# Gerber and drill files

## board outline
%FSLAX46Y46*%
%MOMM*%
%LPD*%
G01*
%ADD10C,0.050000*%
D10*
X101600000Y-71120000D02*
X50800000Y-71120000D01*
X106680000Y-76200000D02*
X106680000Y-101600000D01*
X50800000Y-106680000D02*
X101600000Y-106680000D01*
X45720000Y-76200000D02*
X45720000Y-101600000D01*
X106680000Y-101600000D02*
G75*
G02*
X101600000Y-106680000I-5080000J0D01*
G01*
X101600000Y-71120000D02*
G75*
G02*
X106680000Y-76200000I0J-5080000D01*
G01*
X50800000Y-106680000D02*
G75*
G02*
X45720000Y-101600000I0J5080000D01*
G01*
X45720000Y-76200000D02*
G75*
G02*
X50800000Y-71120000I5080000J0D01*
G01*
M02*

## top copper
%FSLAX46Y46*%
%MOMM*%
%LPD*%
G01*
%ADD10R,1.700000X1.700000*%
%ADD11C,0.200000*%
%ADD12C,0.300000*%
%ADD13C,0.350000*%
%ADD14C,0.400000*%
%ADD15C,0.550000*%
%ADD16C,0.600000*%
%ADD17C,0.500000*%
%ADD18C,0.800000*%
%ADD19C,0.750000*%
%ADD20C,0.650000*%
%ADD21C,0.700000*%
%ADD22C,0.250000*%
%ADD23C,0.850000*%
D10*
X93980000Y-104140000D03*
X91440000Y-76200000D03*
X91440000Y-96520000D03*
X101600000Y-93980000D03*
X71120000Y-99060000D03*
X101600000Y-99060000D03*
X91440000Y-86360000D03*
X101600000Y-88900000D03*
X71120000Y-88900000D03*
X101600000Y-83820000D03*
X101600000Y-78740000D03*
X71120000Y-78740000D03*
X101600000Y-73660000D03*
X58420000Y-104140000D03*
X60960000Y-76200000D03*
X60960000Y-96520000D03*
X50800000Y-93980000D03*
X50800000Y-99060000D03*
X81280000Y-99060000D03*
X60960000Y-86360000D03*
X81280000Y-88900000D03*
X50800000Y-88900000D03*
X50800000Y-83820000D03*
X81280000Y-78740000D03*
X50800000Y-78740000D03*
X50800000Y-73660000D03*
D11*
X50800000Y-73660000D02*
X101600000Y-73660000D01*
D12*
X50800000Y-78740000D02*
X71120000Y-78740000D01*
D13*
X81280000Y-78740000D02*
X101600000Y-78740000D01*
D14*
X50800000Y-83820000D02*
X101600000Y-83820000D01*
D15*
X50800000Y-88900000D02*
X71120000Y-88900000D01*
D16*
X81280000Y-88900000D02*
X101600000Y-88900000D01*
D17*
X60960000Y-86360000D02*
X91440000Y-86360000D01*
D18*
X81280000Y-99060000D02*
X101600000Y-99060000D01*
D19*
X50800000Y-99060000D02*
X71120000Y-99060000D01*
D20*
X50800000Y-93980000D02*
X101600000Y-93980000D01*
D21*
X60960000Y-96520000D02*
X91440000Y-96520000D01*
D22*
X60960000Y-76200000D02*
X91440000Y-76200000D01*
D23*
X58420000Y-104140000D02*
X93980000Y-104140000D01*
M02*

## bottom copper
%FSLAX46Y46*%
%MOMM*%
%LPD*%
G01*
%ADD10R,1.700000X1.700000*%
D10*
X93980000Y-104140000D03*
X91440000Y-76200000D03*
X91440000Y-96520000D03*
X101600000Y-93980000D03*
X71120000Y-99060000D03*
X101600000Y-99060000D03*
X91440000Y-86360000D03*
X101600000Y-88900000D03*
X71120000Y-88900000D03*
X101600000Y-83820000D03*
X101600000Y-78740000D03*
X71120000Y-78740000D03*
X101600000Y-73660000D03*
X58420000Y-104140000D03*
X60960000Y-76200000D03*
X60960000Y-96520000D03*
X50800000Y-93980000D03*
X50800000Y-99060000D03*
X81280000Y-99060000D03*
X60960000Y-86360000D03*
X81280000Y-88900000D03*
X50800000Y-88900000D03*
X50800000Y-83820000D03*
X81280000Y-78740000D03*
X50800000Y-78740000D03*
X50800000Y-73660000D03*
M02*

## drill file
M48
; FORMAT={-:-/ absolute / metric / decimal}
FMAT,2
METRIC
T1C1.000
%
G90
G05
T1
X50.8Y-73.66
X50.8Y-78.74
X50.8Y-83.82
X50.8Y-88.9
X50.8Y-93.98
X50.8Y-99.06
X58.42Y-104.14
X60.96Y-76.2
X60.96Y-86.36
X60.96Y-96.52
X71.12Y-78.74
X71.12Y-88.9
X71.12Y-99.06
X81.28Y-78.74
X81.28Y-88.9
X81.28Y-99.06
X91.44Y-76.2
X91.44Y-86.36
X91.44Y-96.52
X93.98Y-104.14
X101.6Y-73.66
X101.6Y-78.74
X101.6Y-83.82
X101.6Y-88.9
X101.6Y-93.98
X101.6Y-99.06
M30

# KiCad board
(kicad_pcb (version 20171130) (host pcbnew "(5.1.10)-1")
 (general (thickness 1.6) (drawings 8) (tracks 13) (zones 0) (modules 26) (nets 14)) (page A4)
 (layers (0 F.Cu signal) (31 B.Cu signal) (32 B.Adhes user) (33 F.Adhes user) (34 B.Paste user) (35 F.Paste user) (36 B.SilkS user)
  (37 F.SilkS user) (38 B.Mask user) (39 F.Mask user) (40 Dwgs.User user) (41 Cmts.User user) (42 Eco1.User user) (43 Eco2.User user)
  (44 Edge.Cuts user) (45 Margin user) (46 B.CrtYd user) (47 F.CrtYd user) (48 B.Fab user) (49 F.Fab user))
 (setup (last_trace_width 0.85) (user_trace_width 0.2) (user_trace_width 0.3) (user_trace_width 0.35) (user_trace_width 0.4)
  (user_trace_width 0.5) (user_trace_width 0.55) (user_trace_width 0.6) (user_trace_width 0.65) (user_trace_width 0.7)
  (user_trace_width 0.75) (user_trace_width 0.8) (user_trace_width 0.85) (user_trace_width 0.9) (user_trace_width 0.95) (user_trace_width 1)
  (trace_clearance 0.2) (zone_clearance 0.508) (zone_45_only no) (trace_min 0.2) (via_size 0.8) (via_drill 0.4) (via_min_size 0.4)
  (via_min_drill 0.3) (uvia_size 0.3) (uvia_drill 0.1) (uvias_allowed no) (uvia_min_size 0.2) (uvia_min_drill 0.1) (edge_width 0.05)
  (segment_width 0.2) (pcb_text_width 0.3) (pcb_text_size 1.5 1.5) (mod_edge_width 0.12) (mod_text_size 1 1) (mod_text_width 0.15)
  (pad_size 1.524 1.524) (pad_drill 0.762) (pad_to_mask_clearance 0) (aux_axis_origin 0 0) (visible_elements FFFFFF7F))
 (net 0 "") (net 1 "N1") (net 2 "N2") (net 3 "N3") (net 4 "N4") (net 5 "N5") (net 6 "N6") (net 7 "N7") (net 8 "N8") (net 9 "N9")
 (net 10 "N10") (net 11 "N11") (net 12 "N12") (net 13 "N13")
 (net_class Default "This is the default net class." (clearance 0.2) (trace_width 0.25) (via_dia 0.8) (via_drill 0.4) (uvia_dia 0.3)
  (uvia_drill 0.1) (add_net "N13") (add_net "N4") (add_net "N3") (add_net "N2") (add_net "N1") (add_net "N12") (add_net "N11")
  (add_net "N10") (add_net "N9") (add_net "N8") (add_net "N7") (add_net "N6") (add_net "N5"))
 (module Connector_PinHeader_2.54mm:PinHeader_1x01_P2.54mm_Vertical (layer F.Cu) (at 93.98 104.14)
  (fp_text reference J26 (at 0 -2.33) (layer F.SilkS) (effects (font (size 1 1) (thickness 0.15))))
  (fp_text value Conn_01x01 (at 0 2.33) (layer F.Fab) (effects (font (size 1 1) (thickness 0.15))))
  (pad 1 thru_hole rect (at 0 0) (size 1.7 1.7) (drill 1) (layers *.Cu *.Mask) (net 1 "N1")))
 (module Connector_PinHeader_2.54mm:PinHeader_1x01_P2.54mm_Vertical (layer F.Cu) (at 91.44 76.2)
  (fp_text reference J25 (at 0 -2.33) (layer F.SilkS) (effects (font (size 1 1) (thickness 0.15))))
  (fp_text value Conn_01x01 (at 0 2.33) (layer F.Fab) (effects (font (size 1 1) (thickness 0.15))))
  (pad 1 thru_hole rect (at 0 0) (size 1.7 1.7) (drill 1) (layers *.Cu *.Mask) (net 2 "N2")))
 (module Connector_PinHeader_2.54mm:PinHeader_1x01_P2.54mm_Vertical (layer F.Cu) (at 91.44 96.52)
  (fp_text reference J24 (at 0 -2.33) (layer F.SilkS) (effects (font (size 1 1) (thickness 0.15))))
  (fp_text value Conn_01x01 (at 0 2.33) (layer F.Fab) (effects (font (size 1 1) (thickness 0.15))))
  (pad 1 thru_hole rect (at 0 0) (size 1.7 1.7) (drill 1) (layers *.Cu *.Mask) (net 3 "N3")))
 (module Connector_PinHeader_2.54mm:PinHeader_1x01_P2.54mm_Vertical (layer F.Cu) (at 101.6 93.98)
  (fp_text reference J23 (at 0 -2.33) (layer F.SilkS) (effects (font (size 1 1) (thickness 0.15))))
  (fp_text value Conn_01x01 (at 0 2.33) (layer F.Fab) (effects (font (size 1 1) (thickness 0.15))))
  (pad 1 thru_hole rect (at 0 0) (size 1.7 1.7) (drill 1) (layers *.Cu *.Mask) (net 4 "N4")))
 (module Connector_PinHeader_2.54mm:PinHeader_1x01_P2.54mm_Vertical (layer F.Cu) (at 71.12 99.06)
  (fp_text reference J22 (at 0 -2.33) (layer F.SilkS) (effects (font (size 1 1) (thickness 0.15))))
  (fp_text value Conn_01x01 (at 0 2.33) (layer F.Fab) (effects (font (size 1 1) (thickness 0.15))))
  (pad 1 thru_hole rect (at 0 0) (size 1.7 1.7) (drill 1) (layers *.Cu *.Mask) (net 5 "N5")))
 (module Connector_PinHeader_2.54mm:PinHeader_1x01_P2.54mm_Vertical (layer F.Cu) (at 101.6 99.06)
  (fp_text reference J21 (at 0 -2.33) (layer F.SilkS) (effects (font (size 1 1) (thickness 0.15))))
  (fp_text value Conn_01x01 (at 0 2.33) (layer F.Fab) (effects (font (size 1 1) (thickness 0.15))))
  (pad 1 thru_hole rect (at 0 0) (size 1.7 1.7) (drill 1) (layers *.Cu *.Mask) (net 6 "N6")))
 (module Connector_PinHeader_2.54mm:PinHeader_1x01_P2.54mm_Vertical (layer F.Cu) (at 91.44 86.36)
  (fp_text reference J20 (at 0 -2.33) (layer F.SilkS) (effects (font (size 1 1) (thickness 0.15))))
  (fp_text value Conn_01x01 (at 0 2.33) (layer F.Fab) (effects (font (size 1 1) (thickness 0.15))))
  (pad 1 thru_hole rect (at 0 0) (size 1.7 1.7) (drill 1) (layers *.Cu *.Mask) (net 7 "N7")))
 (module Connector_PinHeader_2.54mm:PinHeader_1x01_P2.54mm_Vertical (layer F.Cu) (at 101.6 88.9)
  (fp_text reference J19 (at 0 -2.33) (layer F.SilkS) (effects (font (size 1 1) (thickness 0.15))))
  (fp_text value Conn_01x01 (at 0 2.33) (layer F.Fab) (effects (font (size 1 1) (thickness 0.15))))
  (pad 1 thru_hole rect (at 0 0) (size 1.7 1.7) (drill 1) (layers *.Cu *.Mask) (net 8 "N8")))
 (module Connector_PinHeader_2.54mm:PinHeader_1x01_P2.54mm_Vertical (layer F.Cu) (at 71.12 88.9)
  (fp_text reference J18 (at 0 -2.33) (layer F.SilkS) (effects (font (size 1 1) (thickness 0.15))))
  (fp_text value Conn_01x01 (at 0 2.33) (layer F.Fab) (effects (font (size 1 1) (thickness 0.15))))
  (pad 1 thru_hole rect (at 0 0) (size 1.7 1.7) (drill 1) (layers *.Cu *.Mask) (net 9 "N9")))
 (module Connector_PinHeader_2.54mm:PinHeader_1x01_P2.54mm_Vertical (layer F.Cu) (at 101.6 83.82)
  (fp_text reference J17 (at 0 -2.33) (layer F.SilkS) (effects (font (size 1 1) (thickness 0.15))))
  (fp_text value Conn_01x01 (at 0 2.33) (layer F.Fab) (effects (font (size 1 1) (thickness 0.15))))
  (pad 1 thru_hole rect (at 0 0) (size 1.7 1.7) (drill 1) (layers *.Cu *.Mask) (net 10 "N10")))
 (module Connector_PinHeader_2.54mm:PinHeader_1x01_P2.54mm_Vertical (layer F.Cu) (at 101.6 78.74)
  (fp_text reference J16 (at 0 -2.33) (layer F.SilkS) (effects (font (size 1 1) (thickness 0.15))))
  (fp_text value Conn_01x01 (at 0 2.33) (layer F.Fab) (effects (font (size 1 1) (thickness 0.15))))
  (pad 1 thru_hole rect (at 0 0) (size 1.7 1.7) (drill 1) (layers *.Cu *.Mask) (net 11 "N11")))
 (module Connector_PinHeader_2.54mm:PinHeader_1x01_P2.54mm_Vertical (layer F.Cu) (at 71.12 78.74)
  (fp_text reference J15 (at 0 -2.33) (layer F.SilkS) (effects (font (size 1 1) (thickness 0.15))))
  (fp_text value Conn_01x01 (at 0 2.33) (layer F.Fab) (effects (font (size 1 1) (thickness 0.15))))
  (pad 1 thru_hole rect (at 0 0) (size 1.7 1.7) (drill 1) (layers *.Cu *.Mask) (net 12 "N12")))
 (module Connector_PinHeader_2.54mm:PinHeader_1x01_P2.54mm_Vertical (layer F.Cu) (at 101.6 73.66)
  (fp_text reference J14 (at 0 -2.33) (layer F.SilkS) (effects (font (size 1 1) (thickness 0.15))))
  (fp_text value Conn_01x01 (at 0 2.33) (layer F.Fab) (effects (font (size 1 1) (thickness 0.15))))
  (pad 1 thru_hole rect (at 0 0) (size 1.7 1.7) (drill 1) (layers *.Cu *.Mask) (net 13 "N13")))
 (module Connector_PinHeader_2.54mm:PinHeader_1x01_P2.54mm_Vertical (layer F.Cu) (at 58.42 104.14)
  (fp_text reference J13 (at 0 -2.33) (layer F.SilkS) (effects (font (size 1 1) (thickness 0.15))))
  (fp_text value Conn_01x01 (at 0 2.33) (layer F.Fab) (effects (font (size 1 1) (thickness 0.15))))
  (pad 1 thru_hole rect (at 0 0) (size 1.7 1.7) (drill 1) (layers *.Cu *.Mask) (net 1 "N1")))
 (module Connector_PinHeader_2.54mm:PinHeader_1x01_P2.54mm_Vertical (layer F.Cu) (at 60.96 76.2)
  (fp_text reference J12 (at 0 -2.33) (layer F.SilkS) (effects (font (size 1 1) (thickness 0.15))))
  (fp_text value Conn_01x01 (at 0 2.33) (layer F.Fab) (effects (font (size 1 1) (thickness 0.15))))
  (pad 1 thru_hole rect (at 0 0) (size 1.7 1.7) (drill 1) (layers *.Cu *.Mask) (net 2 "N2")))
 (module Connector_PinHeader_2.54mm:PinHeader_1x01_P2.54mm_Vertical (layer F.Cu) (at 60.96 96.52)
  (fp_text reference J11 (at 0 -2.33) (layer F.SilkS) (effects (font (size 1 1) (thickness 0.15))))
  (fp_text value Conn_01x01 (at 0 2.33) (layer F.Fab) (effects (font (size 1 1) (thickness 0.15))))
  (pad 1 thru_hole rect (at 0 0) (size 1.7 1.7) (drill 1) (layers *.Cu *.Mask) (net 3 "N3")))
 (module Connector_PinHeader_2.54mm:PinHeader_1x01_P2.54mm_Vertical (layer F.Cu) (at 50.8 93.98)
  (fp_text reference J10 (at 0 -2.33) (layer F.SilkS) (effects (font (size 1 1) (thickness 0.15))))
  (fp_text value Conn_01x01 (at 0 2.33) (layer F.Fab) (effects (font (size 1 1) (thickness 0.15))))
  (pad 1 thru_hole rect (at 0 0) (size 1.7 1.7) (drill 1) (layers *.Cu *.Mask) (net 4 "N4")))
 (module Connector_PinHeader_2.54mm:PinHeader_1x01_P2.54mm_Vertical (layer F.Cu) (at 50.8 99.06)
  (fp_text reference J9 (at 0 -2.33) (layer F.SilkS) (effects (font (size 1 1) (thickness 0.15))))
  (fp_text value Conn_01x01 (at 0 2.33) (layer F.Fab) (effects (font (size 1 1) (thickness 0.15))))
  (pad 1 thru_hole rect (at 0 0) (size 1.7 1.7) (drill 1) (layers *.Cu *.Mask) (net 5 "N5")))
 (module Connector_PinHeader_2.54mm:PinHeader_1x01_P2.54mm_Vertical (layer F.Cu) (at 81.28 99.06)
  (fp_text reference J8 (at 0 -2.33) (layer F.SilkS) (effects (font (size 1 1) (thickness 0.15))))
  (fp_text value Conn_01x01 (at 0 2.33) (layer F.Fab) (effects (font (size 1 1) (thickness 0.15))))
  (pad 1 thru_hole rect (at 0 0) (size 1.7 1.7) (drill 1) (layers *.Cu *.Mask) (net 6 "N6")))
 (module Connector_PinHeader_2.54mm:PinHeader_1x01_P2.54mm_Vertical (layer F.Cu) (at 60.96 86.36)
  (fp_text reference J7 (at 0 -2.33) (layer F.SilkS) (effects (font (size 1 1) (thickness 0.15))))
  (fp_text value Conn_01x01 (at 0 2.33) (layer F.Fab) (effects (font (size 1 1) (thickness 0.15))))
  (pad 1 thru_hole rect (at 0 0) (size 1.7 1.7) (drill 1) (layers *.Cu *.Mask) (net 7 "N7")))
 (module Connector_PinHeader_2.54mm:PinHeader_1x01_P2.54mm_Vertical (layer F.Cu) (at 81.28 88.9)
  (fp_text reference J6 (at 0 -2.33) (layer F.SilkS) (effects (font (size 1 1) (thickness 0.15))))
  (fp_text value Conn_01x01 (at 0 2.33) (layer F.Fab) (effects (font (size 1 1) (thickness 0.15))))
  (pad 1 thru_hole rect (at 0 0) (size 1.7 1.7) (drill 1) (layers *.Cu *.Mask) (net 8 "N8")))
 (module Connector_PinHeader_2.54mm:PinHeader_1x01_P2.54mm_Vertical (layer F.Cu) (at 50.8 88.9)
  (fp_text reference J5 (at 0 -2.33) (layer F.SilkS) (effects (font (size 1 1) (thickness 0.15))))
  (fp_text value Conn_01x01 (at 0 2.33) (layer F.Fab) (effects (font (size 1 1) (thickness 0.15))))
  (pad 1 thru_hole rect (at 0 0) (size 1.7 1.7) (drill 1) (layers *.Cu *.Mask) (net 9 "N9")))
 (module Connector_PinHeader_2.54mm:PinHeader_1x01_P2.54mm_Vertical (layer F.Cu) (at 50.8 83.82)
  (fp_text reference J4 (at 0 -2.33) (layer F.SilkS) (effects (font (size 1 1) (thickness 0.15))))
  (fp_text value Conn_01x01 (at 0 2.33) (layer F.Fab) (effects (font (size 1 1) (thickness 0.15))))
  (pad 1 thru_hole rect (at 0 0) (size 1.7 1.7) (drill 1) (layers *.Cu *.Mask) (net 10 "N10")))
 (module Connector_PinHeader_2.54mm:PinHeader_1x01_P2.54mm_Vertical (layer F.Cu) (at 81.28 78.74)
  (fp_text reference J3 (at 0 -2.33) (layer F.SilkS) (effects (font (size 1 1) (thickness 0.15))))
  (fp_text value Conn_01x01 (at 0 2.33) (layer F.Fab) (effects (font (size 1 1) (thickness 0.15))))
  (pad 1 thru_hole rect (at 0 0) (size 1.7 1.7) (drill 1) (layers *.Cu *.Mask) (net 11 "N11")))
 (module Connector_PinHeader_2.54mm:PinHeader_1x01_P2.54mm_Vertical (layer F.Cu) (at 50.8 78.74)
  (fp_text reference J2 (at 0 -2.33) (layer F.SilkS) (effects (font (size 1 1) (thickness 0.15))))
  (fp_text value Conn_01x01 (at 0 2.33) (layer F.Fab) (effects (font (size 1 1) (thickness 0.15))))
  (pad 1 thru_hole rect (at 0 0) (size 1.7 1.7) (drill 1) (layers *.Cu *.Mask) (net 12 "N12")))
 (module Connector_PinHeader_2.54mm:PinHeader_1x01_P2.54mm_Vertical (layer F.Cu) (at 50.8 73.66)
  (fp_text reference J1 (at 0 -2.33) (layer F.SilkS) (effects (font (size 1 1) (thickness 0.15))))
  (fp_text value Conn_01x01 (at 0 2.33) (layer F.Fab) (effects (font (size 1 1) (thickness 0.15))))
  (pad 1 thru_hole rect (at 0 0) (size 1.7 1.7) (drill 1) (layers *.Cu *.Mask) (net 13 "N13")))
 (gr_line (start 101.6 71.12) (end 50.8 71.12) (layer Edge.Cuts) (width 0.05))
 (gr_line (start 106.68 76.2) (end 106.68 101.6) (layer Edge.Cuts) (width 0.05))
 (gr_line (start 50.8 106.68) (end 101.6 106.68) (layer Edge.Cuts) (width 0.05))
 (gr_line (start 45.72 76.2) (end 45.72 101.6) (layer Edge.Cuts) (width 0.05))
 (gr_arc (start 101.6 101.6) (end 101.6 106.68) (angle -90) (layer Edge.Cuts) (width 0.05))
 (gr_arc (start 101.6 76.2) (end 106.68 76.2) (angle -90) (layer Edge.Cuts) (width 0.05))
 (gr_arc (start 50.8 101.6) (end 45.72 101.6) (angle -90) (layer Edge.Cuts) (width 0.05))
 (gr_arc (start 50.8 76.2) (end 50.8 71.12) (angle -90) (layer Edge.Cuts) (width 0.05))
 (segment (start 50.8 73.66) (end 101.6 73.66) (width 0.2) (layer F.Cu) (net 13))
 (segment (start 50.8 78.74) (end 71.12 78.74) (width 0.3) (layer F.Cu) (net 12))
 (segment (start 81.28 78.74) (end 101.6 78.74) (width 0.35) (layer F.Cu) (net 11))
 (segment (start 50.8 83.82) (end 101.6 83.82) (width 0.4) (layer F.Cu) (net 10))
 (segment (start 50.8 88.9) (end 71.12 88.9) (width 0.55) (layer F.Cu) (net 9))
 (segment (start 81.28 88.9) (end 101.6 88.9) (width 0.6) (layer F.Cu) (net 8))
 (segment (start 60.96 86.36) (end 91.44 86.36) (width 0.5) (layer F.Cu) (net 7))
 (segment (start 81.28 99.06) (end 101.6 99.06) (width 0.8) (layer F.Cu) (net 6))
 (segment (start 50.8 99.06) (end 71.12 99.06) (width 0.75) (layer F.Cu) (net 5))
 (segment (start 50.8 93.98) (end 101.6 93.98) (width 0.65) (layer F.Cu) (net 4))
 (segment (start 60.96 96.52) (end 91.44 96.52) (width 0.7) (layer F.Cu) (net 3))
 (segment (start 60.96 76.2) (end 91.44 76.2) (width 0.25) (layer F.Cu) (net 2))
 (segment (start 58.42 104.14) (end 93.98 104.14) (width 0.85) (layer F.Cu) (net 1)))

